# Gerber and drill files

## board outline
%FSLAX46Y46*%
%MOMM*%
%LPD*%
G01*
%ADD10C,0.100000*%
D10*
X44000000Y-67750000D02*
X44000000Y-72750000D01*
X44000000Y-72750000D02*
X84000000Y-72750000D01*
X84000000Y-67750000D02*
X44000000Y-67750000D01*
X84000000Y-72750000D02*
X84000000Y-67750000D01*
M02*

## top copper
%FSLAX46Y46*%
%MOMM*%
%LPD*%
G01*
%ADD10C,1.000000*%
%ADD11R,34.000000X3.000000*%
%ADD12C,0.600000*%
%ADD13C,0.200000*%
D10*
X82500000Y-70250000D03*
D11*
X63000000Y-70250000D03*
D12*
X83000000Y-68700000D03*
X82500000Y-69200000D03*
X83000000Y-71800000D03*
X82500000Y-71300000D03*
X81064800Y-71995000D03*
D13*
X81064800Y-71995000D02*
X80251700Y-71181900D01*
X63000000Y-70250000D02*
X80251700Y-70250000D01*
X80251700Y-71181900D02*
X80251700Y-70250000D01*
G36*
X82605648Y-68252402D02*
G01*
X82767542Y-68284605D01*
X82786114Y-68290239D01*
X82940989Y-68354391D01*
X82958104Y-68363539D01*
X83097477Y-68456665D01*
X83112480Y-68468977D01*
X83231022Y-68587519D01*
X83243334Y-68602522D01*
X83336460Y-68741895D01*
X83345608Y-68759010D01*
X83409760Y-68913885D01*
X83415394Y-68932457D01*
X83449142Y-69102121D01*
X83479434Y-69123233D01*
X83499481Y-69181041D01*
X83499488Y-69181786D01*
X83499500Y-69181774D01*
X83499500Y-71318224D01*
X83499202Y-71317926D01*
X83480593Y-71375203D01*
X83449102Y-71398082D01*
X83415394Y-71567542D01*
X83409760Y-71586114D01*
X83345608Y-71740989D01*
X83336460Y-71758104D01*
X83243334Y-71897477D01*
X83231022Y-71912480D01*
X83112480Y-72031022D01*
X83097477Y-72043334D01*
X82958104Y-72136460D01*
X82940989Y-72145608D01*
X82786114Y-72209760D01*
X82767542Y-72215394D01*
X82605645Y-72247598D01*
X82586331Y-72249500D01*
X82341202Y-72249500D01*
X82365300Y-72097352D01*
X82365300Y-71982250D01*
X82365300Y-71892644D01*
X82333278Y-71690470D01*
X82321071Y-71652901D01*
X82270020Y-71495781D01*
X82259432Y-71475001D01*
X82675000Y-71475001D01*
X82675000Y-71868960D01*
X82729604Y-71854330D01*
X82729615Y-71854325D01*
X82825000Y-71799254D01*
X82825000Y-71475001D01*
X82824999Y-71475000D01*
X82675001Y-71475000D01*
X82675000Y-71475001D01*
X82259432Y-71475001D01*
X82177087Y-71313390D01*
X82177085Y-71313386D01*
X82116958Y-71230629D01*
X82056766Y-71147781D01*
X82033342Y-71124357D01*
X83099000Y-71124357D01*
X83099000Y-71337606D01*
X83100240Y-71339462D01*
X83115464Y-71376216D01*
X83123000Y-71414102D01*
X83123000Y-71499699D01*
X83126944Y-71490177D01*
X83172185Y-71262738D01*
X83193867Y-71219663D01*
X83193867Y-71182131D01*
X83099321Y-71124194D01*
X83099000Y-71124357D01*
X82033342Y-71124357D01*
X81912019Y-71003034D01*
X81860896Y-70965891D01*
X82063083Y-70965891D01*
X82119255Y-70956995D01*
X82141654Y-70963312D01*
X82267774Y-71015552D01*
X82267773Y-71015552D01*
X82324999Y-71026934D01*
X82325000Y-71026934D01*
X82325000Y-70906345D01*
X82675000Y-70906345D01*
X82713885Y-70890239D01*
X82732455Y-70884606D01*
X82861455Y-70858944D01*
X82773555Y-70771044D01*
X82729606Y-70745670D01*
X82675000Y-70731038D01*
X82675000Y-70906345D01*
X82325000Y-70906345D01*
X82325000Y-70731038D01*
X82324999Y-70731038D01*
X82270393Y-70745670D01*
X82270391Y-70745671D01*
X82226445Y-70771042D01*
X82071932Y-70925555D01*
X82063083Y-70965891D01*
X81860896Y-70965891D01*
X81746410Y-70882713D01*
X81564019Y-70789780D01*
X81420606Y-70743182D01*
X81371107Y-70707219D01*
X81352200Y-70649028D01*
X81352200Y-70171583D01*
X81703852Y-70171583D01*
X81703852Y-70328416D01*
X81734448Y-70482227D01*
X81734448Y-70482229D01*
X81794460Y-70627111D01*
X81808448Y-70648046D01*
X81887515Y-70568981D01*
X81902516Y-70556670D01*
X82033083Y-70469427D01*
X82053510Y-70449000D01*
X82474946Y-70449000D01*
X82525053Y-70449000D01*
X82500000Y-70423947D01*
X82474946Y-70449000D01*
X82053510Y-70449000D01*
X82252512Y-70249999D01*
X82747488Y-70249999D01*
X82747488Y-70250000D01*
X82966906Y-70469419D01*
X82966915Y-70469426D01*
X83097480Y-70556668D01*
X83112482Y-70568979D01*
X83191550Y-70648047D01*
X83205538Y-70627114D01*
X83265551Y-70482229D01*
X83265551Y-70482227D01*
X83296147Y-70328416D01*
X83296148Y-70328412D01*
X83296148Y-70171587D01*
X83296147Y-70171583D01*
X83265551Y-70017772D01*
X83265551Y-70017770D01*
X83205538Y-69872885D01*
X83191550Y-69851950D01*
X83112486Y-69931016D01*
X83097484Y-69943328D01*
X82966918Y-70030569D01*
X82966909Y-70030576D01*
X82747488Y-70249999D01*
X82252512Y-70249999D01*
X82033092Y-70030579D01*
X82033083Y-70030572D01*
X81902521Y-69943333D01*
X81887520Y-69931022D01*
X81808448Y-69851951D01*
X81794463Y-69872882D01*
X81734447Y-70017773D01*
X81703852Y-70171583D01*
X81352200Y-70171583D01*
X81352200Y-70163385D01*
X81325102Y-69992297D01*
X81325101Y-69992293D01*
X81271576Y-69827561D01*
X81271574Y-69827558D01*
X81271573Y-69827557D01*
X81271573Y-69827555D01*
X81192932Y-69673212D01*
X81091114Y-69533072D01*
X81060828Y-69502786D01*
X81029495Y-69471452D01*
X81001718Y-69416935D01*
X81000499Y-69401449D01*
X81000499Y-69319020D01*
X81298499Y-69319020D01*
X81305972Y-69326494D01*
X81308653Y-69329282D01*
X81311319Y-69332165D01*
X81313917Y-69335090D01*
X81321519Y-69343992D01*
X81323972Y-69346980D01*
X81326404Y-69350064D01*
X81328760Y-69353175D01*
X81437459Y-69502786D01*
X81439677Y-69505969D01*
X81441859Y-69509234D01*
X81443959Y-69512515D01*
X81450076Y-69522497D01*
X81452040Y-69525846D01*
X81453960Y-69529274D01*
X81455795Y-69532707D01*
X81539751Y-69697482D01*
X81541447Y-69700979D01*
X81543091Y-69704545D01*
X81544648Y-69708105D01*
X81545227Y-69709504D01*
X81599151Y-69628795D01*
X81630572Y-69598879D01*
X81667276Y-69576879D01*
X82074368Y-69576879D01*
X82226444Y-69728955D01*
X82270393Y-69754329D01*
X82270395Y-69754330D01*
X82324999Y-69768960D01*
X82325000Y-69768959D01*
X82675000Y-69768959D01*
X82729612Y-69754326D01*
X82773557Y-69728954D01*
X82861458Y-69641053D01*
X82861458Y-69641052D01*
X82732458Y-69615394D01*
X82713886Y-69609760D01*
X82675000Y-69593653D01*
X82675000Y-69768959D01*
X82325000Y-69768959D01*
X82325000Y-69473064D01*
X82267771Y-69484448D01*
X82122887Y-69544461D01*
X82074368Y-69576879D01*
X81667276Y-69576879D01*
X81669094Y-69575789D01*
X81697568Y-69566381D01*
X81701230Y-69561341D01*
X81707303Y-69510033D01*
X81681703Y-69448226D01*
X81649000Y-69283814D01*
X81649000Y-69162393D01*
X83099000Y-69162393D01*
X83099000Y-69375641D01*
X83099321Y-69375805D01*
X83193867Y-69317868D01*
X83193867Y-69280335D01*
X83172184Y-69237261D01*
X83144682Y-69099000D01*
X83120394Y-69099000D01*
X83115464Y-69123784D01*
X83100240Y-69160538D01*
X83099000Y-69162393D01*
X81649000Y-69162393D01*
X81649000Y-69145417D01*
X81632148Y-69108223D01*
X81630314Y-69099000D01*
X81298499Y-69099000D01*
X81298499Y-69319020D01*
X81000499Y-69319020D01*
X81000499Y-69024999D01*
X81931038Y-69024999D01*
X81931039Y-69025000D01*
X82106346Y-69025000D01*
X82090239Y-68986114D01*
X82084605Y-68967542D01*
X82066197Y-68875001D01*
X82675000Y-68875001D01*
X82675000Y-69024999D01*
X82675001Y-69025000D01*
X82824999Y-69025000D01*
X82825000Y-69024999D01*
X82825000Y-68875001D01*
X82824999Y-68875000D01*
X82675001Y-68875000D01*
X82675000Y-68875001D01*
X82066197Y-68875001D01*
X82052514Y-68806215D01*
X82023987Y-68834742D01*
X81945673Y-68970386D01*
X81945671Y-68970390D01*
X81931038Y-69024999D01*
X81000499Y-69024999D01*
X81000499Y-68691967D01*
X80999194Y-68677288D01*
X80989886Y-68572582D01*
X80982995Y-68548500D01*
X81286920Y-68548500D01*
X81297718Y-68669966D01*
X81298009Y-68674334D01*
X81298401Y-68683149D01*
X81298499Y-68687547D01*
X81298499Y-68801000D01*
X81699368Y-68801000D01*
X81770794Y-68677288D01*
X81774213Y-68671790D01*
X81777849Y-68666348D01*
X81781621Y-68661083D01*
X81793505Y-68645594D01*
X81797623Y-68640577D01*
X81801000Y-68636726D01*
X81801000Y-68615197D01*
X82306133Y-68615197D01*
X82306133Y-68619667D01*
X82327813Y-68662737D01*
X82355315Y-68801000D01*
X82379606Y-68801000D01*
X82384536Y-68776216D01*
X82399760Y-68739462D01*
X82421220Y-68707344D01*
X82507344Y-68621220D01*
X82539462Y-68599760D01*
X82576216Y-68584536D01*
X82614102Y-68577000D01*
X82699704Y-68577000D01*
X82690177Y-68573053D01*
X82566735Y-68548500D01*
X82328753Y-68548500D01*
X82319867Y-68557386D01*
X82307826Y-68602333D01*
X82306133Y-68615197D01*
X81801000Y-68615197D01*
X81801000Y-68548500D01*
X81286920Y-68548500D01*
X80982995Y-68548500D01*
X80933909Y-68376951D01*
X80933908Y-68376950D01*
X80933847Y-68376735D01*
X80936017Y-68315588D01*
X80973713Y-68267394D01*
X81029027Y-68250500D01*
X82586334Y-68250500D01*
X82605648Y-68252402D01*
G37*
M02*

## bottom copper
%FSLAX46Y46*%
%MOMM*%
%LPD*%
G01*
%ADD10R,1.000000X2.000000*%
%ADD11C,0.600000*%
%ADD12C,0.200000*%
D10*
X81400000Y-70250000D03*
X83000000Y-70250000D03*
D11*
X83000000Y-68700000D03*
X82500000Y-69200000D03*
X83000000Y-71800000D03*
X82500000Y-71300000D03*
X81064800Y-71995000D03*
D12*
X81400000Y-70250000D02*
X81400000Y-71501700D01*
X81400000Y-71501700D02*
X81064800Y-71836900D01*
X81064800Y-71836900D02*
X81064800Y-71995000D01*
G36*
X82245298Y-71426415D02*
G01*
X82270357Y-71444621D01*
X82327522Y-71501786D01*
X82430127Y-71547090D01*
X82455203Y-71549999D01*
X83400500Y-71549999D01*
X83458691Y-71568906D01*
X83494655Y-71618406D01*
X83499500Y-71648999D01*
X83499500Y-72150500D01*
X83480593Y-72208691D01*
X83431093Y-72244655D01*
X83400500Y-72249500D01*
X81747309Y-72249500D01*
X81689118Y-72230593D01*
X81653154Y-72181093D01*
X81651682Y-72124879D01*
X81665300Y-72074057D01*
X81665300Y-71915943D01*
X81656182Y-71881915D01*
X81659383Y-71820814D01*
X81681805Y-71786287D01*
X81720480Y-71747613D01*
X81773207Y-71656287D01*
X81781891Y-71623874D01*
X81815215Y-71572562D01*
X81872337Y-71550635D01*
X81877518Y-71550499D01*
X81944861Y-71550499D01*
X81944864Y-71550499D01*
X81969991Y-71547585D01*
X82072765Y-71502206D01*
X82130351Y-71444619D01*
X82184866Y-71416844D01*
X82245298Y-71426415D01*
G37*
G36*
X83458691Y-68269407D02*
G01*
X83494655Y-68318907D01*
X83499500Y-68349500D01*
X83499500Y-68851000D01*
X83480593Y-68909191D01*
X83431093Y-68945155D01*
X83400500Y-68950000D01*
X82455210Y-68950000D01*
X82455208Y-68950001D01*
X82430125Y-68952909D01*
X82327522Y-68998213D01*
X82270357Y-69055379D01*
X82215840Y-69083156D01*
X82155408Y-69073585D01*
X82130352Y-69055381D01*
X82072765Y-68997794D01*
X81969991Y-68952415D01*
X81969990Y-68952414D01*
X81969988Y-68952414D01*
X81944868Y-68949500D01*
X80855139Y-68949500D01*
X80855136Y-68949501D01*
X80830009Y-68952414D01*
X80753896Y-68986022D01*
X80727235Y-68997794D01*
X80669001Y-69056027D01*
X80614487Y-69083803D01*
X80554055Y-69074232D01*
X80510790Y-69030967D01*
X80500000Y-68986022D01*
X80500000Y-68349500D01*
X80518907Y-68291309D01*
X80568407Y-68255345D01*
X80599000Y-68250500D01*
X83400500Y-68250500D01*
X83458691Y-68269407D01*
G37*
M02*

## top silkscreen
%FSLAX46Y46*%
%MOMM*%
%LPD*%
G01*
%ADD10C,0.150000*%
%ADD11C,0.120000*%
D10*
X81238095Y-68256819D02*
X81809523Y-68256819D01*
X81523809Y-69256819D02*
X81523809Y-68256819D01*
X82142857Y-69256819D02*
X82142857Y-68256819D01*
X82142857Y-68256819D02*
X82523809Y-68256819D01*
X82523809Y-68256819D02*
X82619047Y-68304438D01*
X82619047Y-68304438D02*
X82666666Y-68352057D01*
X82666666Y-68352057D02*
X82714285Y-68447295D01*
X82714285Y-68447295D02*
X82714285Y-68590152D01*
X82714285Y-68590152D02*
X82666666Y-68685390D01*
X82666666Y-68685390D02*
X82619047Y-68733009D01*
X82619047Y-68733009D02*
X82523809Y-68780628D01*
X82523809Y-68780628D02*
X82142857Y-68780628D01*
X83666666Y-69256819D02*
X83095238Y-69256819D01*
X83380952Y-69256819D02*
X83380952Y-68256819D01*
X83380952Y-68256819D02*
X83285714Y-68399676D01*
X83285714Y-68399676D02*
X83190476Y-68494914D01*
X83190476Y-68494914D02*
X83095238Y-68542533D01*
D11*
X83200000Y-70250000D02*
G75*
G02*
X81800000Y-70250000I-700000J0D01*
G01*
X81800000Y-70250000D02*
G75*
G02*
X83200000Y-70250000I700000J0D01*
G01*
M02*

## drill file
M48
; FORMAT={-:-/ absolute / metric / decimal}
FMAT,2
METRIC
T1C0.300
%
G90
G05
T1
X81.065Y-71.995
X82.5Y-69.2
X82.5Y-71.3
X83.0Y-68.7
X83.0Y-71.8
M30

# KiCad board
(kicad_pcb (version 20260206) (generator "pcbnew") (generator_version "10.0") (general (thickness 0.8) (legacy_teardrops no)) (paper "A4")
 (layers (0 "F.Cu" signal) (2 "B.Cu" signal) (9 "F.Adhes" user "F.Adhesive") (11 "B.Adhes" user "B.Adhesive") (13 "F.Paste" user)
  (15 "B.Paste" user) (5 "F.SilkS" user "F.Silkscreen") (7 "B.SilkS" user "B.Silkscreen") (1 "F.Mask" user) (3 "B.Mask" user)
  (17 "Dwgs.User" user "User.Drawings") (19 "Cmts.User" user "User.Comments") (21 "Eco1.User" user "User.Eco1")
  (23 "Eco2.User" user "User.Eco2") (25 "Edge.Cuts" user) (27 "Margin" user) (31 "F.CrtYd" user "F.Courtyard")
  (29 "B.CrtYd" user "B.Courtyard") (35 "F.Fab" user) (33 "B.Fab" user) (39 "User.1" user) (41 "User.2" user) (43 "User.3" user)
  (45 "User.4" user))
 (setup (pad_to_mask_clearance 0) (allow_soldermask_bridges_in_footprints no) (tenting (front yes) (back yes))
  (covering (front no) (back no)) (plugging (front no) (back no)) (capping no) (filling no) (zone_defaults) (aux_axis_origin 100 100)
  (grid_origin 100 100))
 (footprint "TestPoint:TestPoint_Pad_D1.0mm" (layer "F.Cu") (at 82.5 70.25)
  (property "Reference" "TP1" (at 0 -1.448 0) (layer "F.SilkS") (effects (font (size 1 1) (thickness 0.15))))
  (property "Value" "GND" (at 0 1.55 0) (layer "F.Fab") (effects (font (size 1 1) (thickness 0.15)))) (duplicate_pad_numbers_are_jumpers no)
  (fp_circle (center 0 0) (end 0 0.7) (stroke (width 0.12) (type solid)) (fill no) (layer "F.SilkS"))
  (pad "1" smd circle (at 0 0) (size 1 1) (layers "F.Cu" "F.Mask") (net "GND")))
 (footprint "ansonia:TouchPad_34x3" (layer "F.Cu") (at 63 70.25)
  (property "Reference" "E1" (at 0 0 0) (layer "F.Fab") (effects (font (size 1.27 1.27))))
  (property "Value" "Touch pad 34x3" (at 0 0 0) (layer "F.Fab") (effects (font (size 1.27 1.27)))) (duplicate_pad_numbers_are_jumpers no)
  (pad "1" smd rect (at 0 0) (size 34 3) (layers "F.Cu") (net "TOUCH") (thermal_bridge_angle 45)))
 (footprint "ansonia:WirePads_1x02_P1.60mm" (layer "B.Cu") (at 82.2 70.25)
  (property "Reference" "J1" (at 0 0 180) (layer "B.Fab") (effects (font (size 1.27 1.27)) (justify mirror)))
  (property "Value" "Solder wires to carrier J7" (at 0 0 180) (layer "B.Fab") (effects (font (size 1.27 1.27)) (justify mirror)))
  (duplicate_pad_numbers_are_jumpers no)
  (pad "1" smd rect (at -0.8 0) (size 1 2) (layers "B.Cu" "B.Mask") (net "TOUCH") (thermal_bridge_angle 45))
  (pad "2" smd rect (at 0.8 0) (size 1 2) (layers "B.Cu" "B.Mask") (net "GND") (thermal_bridge_angle 45)))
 (gr_line (start 44 67.75) (end 44 72.75) (stroke (width 0.1) (type default)) (layer "Edge.Cuts"))
 (gr_line (start 44 72.75) (end 84 72.75) (stroke (width 0.1) (type default)) (layer "Edge.Cuts"))
 (gr_line (start 84 67.75) (end 44 67.75) (stroke (width 0.1) (type default)) (layer "Edge.Cuts"))
 (gr_line (start 84 72.75) (end 84 67.75) (stroke (width 0.1) (type default)) (layer "Edge.Cuts"))
 (via (at 83 68.7) (size 0.6) (drill 0.3) (layers "F.Cu" "B.Cu") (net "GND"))
 (via (at 82.5 69.2) (size 0.6) (drill 0.3) (layers "F.Cu" "B.Cu") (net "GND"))
 (via (at 83 71.8) (size 0.6) (drill 0.3) (layers "F.Cu" "B.Cu") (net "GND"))
 (via (at 82.5 71.3) (size 0.6) (drill 0.3) (layers "F.Cu" "B.Cu") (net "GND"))
 (segment (start 81.0648 71.995) (end 80.2517 71.1819) (width 0.2) (layer "F.Cu") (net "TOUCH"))
 (segment (start 63 70.25) (end 80.2517 70.25) (width 0.2) (layer "F.Cu") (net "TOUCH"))
 (segment (start 80.2517 71.1819) (end 80.2517 70.25) (width 0.2) (layer "F.Cu") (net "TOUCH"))
 (via (at 81.0648 71.995) (size 0.6) (drill 0.3) (layers "F.Cu" "B.Cu") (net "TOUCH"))
 (segment (start 81.4 70.25) (end 81.4 71.5017) (width 0.2) (layer "B.Cu") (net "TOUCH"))
 (segment (start 81.4 71.5017) (end 81.0648 71.8369) (width 0.2) (layer "B.Cu") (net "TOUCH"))
 (segment (start 81.0648 71.8369) (end 81.0648 71.995) (width 0.2) (layer "B.Cu") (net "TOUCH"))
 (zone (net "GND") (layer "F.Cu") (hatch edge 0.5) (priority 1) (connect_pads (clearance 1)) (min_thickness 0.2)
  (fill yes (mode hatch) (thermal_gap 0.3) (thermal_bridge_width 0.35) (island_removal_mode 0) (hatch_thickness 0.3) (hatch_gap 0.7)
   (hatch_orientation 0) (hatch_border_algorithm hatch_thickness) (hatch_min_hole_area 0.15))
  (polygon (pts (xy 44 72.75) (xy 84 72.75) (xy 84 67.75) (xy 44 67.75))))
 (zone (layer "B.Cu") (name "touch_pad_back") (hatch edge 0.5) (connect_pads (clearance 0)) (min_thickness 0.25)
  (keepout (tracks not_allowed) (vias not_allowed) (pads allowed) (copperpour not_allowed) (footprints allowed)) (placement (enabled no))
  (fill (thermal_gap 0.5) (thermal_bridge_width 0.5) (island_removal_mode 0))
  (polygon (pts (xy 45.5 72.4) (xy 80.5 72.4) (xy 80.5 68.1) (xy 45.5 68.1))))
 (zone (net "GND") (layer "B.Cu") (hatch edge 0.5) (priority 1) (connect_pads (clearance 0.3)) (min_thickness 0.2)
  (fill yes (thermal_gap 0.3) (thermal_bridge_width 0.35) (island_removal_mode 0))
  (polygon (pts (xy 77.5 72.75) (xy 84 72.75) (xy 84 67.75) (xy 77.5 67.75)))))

